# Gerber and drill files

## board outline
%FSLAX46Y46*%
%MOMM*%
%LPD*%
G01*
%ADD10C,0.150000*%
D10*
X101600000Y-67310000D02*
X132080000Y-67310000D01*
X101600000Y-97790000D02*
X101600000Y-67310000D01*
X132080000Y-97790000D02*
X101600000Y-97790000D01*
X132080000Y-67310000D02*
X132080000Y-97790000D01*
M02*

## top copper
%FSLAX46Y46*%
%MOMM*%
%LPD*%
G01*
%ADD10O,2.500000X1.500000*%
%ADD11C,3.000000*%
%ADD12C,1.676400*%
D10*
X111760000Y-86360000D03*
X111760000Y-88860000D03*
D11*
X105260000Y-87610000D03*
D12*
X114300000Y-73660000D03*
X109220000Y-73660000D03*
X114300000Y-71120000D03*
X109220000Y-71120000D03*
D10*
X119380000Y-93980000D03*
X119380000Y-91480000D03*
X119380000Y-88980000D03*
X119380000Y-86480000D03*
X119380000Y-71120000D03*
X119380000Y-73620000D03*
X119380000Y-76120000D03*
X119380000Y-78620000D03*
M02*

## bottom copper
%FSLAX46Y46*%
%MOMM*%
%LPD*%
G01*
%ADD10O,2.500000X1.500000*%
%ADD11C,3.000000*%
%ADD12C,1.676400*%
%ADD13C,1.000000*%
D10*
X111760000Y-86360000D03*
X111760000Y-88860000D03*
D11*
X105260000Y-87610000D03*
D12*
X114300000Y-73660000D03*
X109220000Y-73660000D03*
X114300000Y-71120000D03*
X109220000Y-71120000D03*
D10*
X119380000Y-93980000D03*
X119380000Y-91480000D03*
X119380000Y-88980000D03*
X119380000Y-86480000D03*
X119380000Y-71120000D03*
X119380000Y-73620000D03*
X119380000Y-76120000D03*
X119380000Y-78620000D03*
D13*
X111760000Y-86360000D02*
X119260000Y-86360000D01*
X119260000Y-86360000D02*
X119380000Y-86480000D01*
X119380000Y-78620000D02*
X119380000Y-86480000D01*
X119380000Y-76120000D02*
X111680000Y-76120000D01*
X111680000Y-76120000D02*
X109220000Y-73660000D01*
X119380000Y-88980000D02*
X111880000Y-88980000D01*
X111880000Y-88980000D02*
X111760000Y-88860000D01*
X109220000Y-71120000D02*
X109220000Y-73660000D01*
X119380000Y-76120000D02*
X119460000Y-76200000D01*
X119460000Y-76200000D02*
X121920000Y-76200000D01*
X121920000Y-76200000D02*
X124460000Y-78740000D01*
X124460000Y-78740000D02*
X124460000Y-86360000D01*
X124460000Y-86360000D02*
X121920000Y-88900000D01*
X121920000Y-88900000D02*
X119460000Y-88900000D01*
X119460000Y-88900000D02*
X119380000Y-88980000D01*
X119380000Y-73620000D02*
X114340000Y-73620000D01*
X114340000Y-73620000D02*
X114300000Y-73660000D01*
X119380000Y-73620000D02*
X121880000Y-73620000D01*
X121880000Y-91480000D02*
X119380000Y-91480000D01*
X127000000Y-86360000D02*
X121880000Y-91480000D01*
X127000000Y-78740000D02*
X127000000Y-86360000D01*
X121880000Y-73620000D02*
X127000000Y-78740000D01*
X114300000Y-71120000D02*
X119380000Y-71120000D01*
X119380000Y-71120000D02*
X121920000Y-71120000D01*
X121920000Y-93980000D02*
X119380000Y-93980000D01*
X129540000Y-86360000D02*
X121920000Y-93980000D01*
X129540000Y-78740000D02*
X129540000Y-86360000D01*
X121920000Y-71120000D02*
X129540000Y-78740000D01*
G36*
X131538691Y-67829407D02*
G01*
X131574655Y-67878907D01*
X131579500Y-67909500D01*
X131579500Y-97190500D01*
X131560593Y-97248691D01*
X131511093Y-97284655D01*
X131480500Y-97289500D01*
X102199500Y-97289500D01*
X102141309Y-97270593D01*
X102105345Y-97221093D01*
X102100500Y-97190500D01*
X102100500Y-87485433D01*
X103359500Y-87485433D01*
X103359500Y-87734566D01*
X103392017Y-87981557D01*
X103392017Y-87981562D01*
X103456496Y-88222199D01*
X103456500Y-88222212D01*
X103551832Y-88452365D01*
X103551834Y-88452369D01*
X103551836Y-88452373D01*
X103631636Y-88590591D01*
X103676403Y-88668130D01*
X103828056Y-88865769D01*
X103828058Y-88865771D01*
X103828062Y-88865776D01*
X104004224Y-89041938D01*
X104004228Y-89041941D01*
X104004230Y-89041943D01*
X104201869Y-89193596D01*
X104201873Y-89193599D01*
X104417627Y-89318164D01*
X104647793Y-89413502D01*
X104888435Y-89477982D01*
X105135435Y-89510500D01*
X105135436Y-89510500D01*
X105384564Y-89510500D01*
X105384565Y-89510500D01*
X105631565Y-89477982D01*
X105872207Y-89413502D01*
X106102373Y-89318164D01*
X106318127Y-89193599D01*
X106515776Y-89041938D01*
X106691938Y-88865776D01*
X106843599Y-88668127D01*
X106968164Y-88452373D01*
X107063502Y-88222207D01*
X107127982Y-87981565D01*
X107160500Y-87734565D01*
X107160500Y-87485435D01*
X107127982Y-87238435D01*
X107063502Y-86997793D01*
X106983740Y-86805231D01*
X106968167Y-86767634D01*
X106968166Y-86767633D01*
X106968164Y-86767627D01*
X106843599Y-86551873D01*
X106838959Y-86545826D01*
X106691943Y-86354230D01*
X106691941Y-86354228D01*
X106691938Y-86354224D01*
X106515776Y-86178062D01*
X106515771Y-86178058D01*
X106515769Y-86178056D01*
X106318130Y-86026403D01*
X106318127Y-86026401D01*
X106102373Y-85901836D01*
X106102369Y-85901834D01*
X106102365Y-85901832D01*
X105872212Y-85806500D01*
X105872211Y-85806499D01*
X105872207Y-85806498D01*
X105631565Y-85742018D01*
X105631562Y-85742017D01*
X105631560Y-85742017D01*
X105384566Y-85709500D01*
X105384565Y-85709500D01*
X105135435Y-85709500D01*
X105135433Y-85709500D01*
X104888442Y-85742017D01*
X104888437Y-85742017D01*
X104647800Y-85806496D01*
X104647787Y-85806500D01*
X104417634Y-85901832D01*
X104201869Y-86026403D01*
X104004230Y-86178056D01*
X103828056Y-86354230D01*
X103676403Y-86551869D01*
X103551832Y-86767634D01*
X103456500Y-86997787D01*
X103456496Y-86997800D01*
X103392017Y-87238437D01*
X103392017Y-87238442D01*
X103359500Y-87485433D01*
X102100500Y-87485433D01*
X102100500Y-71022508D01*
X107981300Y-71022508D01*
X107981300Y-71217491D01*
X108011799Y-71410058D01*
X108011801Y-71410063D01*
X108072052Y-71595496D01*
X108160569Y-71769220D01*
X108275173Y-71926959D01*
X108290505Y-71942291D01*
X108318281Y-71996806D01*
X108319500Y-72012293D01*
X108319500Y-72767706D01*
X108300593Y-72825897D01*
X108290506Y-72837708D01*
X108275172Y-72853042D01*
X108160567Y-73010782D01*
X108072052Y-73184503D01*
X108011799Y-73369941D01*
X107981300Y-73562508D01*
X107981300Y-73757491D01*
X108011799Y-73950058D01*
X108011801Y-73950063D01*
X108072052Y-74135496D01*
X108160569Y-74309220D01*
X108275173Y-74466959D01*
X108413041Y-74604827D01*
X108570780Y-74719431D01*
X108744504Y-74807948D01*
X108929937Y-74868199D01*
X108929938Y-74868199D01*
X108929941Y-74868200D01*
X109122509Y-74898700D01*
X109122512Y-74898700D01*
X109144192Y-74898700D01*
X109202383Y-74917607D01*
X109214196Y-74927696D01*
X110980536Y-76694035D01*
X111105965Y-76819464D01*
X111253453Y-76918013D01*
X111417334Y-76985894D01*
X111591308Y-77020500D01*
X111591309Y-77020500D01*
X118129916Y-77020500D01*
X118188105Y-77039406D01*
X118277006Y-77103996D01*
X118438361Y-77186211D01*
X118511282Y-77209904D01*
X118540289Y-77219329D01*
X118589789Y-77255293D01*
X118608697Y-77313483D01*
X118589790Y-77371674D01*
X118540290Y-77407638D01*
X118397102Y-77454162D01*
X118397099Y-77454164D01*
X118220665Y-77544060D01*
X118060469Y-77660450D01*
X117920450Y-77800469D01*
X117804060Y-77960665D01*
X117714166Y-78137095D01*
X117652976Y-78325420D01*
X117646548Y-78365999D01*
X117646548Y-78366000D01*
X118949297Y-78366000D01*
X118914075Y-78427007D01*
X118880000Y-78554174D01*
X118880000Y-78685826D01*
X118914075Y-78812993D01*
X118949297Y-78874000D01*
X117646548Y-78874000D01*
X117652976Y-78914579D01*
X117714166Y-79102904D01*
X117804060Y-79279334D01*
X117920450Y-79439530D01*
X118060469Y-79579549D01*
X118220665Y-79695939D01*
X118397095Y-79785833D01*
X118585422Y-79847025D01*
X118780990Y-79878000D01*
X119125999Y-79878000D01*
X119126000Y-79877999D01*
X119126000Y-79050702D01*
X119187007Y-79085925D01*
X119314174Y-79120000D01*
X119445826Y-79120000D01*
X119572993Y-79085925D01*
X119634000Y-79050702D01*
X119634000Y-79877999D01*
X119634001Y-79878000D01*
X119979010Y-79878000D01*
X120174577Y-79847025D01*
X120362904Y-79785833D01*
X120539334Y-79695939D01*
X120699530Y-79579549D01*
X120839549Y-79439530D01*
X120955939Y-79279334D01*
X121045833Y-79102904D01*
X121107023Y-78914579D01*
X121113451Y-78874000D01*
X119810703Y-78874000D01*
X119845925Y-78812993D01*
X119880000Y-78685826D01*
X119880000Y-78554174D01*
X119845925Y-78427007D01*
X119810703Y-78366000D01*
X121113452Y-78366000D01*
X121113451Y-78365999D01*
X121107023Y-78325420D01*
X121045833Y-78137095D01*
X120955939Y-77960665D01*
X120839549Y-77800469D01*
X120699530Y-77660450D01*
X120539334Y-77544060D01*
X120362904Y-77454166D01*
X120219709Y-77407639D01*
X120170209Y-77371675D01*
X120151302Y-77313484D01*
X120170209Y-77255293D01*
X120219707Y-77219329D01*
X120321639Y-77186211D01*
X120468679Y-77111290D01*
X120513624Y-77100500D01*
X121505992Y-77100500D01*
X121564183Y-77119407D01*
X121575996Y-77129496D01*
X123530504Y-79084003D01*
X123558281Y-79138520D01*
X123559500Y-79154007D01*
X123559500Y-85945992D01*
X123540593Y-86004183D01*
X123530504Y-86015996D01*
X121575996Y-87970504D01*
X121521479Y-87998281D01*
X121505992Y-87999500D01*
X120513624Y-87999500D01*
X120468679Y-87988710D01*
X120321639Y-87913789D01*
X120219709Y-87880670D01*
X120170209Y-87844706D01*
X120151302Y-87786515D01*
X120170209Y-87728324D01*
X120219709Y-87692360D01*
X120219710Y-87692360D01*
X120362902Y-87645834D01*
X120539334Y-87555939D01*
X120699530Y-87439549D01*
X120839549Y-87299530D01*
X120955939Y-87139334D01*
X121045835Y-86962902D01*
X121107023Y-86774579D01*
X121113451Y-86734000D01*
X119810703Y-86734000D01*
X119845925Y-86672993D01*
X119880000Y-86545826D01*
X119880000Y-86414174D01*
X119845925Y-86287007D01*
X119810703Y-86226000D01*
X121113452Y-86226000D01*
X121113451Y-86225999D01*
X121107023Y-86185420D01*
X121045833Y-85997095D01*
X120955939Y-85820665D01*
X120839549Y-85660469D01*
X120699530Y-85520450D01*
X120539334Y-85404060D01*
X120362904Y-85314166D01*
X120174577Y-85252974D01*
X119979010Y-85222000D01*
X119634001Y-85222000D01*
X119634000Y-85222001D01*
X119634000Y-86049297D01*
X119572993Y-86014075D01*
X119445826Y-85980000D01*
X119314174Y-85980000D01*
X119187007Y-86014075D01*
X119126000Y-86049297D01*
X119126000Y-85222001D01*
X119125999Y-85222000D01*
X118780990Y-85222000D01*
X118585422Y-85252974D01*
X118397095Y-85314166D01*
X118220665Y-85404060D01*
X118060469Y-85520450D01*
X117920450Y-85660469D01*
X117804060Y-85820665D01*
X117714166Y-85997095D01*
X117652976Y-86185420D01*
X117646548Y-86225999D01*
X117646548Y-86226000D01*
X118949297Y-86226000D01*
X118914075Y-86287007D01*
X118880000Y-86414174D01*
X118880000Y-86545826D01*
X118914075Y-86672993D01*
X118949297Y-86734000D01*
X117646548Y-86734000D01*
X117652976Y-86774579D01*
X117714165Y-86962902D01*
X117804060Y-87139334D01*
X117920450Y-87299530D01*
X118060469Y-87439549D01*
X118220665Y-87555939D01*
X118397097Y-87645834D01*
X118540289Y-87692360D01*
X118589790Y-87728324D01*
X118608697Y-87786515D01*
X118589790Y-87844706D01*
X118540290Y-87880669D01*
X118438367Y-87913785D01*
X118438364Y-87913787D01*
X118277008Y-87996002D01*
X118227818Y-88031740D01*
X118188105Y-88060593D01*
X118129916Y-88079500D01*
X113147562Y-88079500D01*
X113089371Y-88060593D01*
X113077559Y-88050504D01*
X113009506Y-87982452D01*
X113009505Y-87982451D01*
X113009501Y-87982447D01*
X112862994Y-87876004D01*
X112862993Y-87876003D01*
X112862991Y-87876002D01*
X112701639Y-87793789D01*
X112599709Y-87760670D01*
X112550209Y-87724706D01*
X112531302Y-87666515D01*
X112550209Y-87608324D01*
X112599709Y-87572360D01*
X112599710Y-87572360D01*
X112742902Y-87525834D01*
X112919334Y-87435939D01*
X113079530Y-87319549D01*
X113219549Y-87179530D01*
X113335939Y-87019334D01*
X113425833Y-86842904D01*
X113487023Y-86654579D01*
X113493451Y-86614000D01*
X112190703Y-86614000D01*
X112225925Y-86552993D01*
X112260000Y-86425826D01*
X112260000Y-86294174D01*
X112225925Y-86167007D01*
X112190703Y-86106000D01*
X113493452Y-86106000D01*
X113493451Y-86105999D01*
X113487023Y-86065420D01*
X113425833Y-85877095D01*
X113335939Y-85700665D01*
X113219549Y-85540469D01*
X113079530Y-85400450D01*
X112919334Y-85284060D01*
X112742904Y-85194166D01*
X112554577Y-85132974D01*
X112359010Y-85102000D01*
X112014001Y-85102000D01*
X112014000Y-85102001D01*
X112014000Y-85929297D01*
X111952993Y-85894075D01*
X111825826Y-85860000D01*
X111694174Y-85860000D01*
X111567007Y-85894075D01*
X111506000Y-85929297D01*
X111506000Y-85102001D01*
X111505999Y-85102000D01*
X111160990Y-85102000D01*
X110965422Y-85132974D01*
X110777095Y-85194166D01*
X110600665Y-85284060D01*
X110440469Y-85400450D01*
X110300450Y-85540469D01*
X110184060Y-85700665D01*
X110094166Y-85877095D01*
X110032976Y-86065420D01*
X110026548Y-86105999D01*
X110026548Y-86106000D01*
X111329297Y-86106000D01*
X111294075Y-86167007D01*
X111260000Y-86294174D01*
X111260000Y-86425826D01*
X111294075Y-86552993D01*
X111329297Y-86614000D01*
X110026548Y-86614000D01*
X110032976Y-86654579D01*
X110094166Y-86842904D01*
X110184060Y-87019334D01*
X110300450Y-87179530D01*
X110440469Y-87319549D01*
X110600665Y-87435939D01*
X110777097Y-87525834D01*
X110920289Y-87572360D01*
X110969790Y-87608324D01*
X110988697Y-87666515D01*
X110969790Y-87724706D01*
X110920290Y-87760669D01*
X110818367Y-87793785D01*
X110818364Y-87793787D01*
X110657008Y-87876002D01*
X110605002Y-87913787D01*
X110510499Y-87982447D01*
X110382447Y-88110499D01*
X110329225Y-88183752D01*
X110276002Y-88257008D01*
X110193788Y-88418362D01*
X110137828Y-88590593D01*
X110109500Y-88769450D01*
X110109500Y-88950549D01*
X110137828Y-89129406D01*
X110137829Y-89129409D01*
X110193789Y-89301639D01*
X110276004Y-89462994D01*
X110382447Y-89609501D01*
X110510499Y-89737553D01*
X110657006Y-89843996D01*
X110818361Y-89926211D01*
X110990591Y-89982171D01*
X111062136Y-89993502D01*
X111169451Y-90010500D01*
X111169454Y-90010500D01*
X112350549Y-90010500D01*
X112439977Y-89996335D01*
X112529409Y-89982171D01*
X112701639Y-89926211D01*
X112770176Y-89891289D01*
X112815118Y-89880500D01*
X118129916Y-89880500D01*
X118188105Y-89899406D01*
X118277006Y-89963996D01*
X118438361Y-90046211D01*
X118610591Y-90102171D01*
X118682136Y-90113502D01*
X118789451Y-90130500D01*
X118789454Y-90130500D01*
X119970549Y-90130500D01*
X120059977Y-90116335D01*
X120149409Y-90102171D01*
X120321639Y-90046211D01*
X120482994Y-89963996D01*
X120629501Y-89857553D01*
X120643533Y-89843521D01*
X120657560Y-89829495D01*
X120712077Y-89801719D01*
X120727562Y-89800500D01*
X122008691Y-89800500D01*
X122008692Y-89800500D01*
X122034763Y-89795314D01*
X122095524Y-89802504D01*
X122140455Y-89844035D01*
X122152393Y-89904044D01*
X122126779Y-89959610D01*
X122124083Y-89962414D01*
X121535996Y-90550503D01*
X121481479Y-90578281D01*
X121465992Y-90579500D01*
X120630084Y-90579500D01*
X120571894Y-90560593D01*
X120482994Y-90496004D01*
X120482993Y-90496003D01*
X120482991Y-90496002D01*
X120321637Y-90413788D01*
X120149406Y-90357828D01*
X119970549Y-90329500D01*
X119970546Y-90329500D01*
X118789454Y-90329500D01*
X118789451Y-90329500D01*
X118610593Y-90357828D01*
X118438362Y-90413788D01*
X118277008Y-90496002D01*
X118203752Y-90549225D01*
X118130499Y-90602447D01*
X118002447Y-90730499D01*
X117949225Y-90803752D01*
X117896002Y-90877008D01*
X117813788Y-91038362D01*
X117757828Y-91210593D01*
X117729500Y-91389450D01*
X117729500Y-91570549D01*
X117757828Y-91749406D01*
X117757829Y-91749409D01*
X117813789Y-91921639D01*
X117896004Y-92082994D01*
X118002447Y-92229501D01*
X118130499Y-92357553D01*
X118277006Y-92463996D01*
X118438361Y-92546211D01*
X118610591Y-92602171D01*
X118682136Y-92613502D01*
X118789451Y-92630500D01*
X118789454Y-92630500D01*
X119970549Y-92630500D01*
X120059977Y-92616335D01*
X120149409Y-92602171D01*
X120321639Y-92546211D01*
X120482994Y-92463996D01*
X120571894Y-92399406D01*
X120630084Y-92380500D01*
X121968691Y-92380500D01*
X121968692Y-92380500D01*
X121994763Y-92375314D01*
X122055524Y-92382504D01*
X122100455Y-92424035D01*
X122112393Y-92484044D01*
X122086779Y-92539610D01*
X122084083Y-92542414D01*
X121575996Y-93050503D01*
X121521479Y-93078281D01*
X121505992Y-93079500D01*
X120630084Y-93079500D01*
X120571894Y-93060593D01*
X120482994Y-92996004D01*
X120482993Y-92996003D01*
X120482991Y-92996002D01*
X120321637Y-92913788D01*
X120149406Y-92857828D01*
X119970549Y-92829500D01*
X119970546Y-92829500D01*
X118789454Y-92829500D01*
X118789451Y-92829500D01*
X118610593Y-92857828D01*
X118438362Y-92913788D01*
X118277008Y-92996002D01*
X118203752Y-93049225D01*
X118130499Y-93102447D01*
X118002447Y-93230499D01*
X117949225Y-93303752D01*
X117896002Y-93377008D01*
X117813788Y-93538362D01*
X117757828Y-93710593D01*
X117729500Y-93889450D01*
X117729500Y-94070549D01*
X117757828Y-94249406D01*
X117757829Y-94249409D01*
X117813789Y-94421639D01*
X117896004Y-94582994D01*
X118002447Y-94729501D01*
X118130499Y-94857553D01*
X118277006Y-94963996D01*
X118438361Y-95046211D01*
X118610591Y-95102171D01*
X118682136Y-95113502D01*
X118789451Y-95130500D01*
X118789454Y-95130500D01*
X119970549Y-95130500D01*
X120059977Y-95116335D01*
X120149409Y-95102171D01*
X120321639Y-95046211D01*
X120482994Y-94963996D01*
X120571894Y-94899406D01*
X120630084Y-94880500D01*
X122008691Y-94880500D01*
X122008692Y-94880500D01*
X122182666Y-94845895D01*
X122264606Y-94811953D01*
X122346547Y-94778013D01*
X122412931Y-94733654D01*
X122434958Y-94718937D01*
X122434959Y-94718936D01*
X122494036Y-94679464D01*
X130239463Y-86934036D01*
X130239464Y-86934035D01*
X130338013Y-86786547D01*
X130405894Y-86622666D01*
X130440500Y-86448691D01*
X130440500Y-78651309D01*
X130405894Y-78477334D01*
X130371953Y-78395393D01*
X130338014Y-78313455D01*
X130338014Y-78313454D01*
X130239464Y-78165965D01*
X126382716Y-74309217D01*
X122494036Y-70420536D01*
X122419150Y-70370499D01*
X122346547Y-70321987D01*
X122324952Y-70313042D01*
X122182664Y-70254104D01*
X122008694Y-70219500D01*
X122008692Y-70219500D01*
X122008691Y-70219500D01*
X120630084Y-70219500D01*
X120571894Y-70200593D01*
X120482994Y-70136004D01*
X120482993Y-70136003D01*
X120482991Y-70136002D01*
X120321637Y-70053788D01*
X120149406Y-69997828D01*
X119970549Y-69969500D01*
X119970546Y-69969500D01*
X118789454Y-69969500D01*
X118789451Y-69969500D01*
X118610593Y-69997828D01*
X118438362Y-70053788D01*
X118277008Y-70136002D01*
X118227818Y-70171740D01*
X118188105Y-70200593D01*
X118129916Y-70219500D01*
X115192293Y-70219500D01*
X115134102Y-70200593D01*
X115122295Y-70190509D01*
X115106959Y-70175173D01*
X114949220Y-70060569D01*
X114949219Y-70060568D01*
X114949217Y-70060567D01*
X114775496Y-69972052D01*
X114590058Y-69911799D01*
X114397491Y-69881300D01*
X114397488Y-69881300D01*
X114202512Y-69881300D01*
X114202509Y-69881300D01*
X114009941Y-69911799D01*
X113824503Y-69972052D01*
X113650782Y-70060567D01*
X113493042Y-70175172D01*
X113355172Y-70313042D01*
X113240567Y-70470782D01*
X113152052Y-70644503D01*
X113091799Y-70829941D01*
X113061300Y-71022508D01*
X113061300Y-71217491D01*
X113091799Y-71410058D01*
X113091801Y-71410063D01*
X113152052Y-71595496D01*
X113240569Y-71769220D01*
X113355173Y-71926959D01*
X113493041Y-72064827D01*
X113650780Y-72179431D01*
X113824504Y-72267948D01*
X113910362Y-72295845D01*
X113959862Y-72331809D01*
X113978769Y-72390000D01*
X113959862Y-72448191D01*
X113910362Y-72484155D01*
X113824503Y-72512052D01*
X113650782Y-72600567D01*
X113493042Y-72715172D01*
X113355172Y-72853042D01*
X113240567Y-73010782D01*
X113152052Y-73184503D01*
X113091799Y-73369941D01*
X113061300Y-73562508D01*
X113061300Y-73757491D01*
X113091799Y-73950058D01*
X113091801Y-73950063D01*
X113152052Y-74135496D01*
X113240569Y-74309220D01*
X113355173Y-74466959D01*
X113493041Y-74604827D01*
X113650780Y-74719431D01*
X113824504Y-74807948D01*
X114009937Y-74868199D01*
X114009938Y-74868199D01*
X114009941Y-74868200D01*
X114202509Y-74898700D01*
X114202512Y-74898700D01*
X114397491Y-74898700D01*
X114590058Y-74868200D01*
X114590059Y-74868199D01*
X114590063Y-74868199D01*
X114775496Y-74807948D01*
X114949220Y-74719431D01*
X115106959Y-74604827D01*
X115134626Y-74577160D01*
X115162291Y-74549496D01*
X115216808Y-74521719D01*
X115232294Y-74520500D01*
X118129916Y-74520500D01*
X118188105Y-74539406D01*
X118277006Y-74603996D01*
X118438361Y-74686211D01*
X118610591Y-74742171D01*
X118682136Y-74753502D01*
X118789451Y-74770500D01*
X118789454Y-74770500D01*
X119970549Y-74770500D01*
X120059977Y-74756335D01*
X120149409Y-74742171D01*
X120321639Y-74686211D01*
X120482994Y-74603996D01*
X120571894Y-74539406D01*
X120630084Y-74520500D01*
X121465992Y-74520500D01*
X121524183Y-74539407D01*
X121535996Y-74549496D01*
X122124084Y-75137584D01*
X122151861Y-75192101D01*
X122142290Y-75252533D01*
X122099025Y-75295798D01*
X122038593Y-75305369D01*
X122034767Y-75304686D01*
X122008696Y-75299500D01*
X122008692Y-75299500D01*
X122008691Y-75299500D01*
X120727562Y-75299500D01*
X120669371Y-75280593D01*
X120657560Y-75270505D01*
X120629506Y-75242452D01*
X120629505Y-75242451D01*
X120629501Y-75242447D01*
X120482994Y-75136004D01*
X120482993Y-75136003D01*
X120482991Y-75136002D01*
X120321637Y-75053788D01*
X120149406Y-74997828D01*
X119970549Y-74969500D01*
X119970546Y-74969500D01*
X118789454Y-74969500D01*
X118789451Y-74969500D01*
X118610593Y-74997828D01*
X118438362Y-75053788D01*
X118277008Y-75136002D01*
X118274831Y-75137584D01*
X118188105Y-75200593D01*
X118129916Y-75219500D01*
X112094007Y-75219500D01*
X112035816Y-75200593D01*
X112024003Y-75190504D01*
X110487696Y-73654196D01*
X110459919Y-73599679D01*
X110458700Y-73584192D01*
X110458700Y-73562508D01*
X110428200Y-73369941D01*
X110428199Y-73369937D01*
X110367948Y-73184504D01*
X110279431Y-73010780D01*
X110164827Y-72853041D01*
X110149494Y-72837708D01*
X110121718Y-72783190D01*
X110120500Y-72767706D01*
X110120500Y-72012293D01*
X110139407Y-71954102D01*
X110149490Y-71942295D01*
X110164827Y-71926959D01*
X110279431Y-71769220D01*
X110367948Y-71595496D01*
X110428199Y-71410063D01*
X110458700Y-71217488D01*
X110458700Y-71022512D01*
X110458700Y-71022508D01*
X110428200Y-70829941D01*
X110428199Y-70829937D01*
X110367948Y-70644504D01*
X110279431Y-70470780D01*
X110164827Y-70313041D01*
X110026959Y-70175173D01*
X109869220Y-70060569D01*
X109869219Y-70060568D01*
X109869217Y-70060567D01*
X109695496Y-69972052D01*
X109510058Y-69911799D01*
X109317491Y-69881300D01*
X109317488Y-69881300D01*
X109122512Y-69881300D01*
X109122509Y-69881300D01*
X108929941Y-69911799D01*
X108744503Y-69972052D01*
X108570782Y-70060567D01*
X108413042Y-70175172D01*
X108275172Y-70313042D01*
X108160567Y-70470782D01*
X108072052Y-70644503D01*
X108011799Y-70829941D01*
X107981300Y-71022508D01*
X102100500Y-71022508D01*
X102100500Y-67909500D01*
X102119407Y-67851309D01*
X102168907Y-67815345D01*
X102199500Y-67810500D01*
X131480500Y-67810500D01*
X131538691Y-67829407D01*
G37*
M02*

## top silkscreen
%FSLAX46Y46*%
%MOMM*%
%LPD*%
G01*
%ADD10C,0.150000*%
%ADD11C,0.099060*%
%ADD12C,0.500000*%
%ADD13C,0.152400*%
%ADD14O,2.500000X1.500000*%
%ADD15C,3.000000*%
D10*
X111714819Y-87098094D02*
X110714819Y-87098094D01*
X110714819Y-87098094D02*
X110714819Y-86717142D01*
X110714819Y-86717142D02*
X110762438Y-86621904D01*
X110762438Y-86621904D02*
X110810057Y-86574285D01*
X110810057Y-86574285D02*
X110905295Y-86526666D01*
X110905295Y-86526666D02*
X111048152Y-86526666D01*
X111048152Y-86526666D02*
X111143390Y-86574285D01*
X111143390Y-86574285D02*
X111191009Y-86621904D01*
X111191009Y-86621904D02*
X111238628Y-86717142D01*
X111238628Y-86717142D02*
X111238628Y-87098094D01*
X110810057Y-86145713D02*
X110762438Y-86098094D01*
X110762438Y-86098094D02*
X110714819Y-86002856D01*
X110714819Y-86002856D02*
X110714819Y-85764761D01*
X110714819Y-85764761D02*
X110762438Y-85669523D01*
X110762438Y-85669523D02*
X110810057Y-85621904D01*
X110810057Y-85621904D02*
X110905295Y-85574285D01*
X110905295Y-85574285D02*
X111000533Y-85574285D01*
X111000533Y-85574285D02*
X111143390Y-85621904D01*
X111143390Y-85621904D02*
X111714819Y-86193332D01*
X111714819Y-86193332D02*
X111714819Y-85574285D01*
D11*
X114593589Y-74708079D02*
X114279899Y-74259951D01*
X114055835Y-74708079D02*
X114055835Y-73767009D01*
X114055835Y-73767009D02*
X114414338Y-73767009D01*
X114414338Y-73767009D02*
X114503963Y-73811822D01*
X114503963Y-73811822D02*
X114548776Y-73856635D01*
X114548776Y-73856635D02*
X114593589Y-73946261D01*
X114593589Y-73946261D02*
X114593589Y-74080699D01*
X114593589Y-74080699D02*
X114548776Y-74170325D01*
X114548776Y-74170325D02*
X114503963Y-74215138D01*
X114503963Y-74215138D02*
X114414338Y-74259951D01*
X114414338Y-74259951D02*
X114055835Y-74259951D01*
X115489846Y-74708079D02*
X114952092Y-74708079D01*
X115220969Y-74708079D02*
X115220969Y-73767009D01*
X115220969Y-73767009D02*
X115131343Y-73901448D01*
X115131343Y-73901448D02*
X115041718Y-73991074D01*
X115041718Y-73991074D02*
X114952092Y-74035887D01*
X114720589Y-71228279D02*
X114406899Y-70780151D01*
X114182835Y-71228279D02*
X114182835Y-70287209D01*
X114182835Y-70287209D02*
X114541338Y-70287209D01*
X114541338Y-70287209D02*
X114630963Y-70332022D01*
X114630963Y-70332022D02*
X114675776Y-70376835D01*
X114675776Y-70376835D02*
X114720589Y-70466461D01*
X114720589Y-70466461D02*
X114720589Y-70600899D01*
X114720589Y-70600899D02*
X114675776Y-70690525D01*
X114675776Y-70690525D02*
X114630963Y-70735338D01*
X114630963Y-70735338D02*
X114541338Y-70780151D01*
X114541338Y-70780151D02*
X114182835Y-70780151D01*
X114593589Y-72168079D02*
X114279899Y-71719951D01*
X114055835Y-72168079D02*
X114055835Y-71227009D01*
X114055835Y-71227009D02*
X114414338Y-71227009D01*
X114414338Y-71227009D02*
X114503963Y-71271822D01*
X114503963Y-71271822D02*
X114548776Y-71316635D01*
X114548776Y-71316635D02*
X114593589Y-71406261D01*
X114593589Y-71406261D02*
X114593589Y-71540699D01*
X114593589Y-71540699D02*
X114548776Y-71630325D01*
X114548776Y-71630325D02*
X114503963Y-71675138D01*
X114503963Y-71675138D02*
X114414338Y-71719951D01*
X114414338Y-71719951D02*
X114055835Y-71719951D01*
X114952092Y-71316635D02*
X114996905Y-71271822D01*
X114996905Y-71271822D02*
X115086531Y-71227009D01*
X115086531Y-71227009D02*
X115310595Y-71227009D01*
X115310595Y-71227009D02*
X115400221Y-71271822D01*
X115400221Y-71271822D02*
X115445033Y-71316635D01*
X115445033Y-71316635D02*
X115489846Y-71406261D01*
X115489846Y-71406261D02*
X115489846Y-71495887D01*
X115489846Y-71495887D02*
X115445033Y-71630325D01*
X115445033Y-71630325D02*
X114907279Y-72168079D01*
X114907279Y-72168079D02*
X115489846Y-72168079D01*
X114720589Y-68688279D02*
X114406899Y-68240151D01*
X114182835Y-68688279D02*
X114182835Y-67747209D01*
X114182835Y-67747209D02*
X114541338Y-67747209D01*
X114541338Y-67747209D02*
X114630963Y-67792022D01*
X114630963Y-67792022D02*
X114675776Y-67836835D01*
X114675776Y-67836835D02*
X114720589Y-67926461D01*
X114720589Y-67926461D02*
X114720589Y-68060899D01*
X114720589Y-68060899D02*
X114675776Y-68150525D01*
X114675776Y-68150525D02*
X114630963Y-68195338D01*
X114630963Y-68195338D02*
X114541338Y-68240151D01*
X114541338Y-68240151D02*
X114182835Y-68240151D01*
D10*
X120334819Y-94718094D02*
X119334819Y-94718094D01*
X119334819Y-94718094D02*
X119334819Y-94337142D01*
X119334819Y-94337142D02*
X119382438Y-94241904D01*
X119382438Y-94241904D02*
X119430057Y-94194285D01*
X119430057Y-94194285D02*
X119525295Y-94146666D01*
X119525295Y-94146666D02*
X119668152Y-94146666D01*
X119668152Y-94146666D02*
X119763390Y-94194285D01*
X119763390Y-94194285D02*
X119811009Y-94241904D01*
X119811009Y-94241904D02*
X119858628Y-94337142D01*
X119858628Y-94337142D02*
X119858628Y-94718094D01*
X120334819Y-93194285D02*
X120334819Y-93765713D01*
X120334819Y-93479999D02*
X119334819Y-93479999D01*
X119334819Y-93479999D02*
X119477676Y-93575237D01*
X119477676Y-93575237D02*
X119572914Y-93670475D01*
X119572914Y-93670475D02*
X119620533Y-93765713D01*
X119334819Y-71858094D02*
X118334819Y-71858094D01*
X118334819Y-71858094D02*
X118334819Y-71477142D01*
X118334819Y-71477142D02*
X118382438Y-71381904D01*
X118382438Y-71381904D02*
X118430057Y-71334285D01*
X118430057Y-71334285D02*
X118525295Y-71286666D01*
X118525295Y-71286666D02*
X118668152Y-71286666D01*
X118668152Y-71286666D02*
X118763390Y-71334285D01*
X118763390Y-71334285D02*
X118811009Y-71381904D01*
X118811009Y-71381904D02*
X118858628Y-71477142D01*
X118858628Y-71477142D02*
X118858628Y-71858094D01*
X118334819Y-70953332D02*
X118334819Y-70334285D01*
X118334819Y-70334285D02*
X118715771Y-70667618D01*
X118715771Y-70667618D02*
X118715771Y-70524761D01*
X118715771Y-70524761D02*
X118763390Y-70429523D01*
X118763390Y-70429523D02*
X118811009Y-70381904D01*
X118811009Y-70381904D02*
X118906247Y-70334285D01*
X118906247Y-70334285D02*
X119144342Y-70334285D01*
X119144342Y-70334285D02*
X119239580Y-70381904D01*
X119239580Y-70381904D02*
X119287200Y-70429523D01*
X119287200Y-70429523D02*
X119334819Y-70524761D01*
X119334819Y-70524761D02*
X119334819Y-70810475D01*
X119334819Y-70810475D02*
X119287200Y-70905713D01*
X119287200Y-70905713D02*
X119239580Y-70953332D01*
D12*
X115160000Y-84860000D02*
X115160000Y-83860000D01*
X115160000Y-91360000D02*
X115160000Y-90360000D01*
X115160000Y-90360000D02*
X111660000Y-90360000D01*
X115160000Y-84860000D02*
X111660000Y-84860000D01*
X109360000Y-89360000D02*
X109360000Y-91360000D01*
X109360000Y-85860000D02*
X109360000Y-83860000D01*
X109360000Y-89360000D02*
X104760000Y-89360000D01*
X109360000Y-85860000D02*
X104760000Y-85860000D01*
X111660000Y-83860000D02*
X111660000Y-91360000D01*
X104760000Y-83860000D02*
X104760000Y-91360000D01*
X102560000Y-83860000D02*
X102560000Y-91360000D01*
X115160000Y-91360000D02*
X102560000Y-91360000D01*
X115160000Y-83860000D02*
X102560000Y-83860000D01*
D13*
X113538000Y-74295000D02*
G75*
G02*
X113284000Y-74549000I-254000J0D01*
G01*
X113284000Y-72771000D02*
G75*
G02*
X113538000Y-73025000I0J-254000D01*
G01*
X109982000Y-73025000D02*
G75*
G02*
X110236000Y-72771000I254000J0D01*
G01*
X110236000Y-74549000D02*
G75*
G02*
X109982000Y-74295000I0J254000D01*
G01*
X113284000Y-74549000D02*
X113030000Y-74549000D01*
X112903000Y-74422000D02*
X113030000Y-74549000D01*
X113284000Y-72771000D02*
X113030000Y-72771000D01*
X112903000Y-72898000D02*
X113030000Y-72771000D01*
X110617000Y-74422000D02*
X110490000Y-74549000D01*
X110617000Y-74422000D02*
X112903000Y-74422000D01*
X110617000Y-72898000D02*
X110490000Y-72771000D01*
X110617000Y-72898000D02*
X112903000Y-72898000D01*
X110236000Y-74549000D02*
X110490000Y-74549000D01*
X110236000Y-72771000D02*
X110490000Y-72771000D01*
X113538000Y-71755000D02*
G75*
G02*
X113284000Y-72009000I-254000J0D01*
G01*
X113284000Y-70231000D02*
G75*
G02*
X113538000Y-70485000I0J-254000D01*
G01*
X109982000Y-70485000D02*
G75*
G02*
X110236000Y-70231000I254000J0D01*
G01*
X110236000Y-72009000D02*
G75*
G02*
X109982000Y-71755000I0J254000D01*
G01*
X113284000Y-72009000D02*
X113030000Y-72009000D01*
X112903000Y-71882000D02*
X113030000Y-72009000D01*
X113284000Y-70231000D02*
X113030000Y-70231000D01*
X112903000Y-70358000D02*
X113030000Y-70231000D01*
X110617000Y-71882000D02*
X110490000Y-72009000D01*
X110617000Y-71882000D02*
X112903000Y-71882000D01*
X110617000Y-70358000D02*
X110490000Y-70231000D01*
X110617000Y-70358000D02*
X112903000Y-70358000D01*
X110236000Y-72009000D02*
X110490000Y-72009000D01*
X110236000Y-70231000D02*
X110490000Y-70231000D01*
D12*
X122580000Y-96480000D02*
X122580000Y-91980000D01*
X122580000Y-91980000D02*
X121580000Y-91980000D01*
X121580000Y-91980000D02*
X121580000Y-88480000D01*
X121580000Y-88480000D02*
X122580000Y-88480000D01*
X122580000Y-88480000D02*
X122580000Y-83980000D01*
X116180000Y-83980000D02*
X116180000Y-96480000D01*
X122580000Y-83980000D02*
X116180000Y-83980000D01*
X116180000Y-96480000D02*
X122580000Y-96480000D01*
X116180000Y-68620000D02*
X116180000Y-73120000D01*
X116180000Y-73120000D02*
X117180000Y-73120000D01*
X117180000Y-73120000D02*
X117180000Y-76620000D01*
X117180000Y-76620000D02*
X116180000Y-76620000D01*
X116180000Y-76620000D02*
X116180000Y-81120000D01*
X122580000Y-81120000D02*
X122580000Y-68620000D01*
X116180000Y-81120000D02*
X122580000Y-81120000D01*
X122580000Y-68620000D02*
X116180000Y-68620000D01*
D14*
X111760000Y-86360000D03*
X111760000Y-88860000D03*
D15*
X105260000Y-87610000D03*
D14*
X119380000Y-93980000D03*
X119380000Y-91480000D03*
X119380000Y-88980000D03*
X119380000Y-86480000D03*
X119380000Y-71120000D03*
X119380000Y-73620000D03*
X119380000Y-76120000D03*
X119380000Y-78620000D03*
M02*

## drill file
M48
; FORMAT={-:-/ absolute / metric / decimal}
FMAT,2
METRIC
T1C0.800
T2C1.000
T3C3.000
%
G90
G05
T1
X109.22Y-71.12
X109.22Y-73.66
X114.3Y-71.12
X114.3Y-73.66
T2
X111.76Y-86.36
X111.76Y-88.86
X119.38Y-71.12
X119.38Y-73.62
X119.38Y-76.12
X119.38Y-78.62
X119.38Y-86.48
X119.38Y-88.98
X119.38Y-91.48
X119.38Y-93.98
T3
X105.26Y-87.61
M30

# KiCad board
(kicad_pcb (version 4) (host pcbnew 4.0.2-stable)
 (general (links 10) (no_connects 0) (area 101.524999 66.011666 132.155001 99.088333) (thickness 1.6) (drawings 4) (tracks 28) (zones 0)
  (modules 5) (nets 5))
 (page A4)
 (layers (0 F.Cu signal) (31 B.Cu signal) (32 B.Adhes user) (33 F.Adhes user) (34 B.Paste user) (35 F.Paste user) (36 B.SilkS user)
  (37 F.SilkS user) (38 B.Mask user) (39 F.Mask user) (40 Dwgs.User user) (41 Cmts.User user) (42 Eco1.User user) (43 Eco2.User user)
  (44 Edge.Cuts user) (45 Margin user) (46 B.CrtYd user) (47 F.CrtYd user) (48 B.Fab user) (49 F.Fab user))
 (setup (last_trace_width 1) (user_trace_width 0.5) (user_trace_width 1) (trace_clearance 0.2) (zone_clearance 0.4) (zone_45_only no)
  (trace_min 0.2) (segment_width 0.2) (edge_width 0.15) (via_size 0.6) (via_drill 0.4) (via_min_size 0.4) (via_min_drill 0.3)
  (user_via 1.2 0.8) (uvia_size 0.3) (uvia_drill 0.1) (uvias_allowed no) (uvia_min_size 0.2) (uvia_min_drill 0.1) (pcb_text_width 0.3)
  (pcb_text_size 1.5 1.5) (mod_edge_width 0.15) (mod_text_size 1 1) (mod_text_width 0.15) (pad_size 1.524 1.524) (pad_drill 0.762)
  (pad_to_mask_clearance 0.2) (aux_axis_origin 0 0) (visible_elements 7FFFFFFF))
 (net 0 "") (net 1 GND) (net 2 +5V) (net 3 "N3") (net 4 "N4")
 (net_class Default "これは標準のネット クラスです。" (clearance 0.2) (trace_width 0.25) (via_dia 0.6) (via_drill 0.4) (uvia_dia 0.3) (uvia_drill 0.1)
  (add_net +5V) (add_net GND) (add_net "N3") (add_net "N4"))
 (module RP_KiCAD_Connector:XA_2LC (layer F.Cu) (at 111.76 86.36 270)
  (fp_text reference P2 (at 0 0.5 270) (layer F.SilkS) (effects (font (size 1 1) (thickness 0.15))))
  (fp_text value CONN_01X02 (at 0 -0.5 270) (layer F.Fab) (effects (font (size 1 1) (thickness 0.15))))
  (fp_line (start -1.5 -3.4) (end -2.5 -3.4) (layer F.SilkS) (width 0.5))
  (fp_line (start 5 -3.4) (end 4 -3.4) (layer F.SilkS) (width 0.5))
  (fp_line (start 4 -3.4) (end 4 0.1) (layer F.SilkS) (width 0.5))
  (fp_line (start -1.5 -3.4) (end -1.5 0.1) (layer F.SilkS) (width 0.5))
  (fp_line (start 3 2.4) (end 5 2.4) (layer F.SilkS) (width 0.5))
  (fp_line (start -0.5 2.4) (end -2.5 2.4) (layer F.SilkS) (width 0.5))
  (fp_line (start 3 2.4) (end 3 7) (layer F.SilkS) (width 0.5))
  (fp_line (start -0.5 2.4) (end -0.5 7) (layer F.SilkS) (width 0.5))
  (fp_line (start -2.5 0.1) (end 5 0.1) (layer F.SilkS) (width 0.5))
  (fp_line (start -2.5 7) (end 5 7) (layer F.SilkS) (width 0.5))
  (fp_line (start -2.5 9.2) (end 5 9.2) (layer F.SilkS) (width 0.5))
  (fp_line (start 5 -3.4) (end 5 9.2) (layer F.SilkS) (width 0.5))
  (fp_line (start -2.5 -3.4) (end -2.5 9.2) (layer F.SilkS) (width 0.5))
  (pad 1 thru_hole oval (at 0 0 270) (size 1.5 2.5) (drill 1) (layers *.Cu *.Mask F.SilkS) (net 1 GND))
  (pad 2 thru_hole oval (at 2.5 0 270) (size 1.5 2.5) (drill 1) (layers *.Cu *.Mask F.SilkS) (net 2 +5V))
  (pad "" thru_hole circle (at 1.25 6.5 270) (size 3 3) (drill 3) (layers *.Cu *.Mask F.SilkS) (clearance -0.3)))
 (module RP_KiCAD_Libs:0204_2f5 (layer F.Cu) (at 111.76 73.66 180)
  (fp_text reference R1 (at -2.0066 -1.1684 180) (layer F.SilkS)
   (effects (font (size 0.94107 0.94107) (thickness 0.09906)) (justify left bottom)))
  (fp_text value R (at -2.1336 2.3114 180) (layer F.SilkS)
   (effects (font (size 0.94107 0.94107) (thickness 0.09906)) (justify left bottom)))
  (fp_arc (start -1.524 -0.635) (end -1.778 -0.635) (angle 90) (layer F.SilkS) (width 0.1524))
  (fp_arc (start -1.524 0.635) (end -1.778 0.635) (angle -90) (layer F.SilkS) (width 0.1524))
  (fp_arc (start 1.524 0.635) (end 1.524 0.889) (angle -90) (layer F.SilkS) (width 0.1524))
  (fp_arc (start 1.524 -0.635) (end 1.524 -0.889) (angle 90) (layer F.SilkS) (width 0.1524))
  (fp_line (start -1.524 -0.889) (end -1.27 -0.889) (layer F.SilkS) (width 0.1524))
  (fp_line (start -1.143 -0.762) (end -1.27 -0.889) (layer F.SilkS) (width 0.1524))
  (fp_line (start -1.524 0.889) (end -1.27 0.889) (layer F.SilkS) (width 0.1524))
  (fp_line (start -1.143 0.762) (end -1.27 0.889) (layer F.SilkS) (width 0.1524))
  (fp_line (start 1.143 -0.762) (end 1.27 -0.889) (layer F.SilkS) (width 0.1524))
  (fp_line (start 1.143 -0.762) (end -1.143 -0.762) (layer F.SilkS) (width 0.1524))
  (fp_line (start 1.143 0.762) (end 1.27 0.889) (layer F.SilkS) (width 0.1524))
  (fp_line (start 1.143 0.762) (end -1.143 0.762) (layer F.SilkS) (width 0.1524))
  (fp_line (start 1.524 -0.889) (end 1.27 -0.889) (layer F.SilkS) (width 0.1524))
  (fp_line (start 1.524 0.889) (end 1.27 0.889) (layer F.SilkS) (width 0.1524))
  (pad 1 thru_hole circle (at -2.54 0 180) (size 1.6764 1.6764) (drill 0.8) (layers *.Cu *.Mask) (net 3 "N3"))
  (pad 2 thru_hole circle (at 2.54 0 180) (size 1.6764 1.6764) (drill 0.8) (layers *.Cu *.Mask) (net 2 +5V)))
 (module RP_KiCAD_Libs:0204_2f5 (layer F.Cu) (at 111.76 71.12 180)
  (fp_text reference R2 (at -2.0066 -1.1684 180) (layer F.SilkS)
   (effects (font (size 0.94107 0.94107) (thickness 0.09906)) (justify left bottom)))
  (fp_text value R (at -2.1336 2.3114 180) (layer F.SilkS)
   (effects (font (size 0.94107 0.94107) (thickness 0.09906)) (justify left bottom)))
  (fp_arc (start -1.524 -0.635) (end -1.778 -0.635) (angle 90) (layer F.SilkS) (width 0.1524))
  (fp_arc (start -1.524 0.635) (end -1.778 0.635) (angle -90) (layer F.SilkS) (width 0.1524))
  (fp_arc (start 1.524 0.635) (end 1.524 0.889) (angle -90) (layer F.SilkS) (width 0.1524))
  (fp_arc (start 1.524 -0.635) (end 1.524 -0.889) (angle 90) (layer F.SilkS) (width 0.1524))
  (fp_line (start -1.524 -0.889) (end -1.27 -0.889) (layer F.SilkS) (width 0.1524))
  (fp_line (start -1.143 -0.762) (end -1.27 -0.889) (layer F.SilkS) (width 0.1524))
  (fp_line (start -1.524 0.889) (end -1.27 0.889) (layer F.SilkS) (width 0.1524))
  (fp_line (start -1.143 0.762) (end -1.27 0.889) (layer F.SilkS) (width 0.1524))
  (fp_line (start 1.143 -0.762) (end 1.27 -0.889) (layer F.SilkS) (width 0.1524))
  (fp_line (start 1.143 -0.762) (end -1.143 -0.762) (layer F.SilkS) (width 0.1524))
  (fp_line (start 1.143 0.762) (end 1.27 0.889) (layer F.SilkS) (width 0.1524))
  (fp_line (start 1.143 0.762) (end -1.143 0.762) (layer F.SilkS) (width 0.1524))
  (fp_line (start 1.524 -0.889) (end 1.27 -0.889) (layer F.SilkS) (width 0.1524))
  (fp_line (start 1.524 0.889) (end 1.27 0.889) (layer F.SilkS) (width 0.1524))
  (pad 1 thru_hole circle (at -2.54 0 180) (size 1.6764 1.6764) (drill 0.8) (layers *.Cu *.Mask) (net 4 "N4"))
  (pad 2 thru_hole circle (at 2.54 0 180) (size 1.6764 1.6764) (drill 0.8) (layers *.Cu *.Mask) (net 2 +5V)))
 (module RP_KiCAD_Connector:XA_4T (layer F.Cu) (at 119.38 93.98 90)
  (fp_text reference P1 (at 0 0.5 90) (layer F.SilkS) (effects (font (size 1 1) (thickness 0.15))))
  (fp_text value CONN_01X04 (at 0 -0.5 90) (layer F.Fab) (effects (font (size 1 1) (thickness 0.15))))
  (fp_line (start -2.5 3.2) (end 2 3.2) (layer F.SilkS) (width 0.5))
  (fp_line (start 2 3.2) (end 2 2.2) (layer F.SilkS) (width 0.5))
  (fp_line (start 2 2.2) (end 5.5 2.2) (layer F.SilkS) (width 0.5))
  (fp_line (start 5.5 2.2) (end 5.5 3.2) (layer F.SilkS) (width 0.5))
  (fp_line (start 5.5 3.2) (end 10 3.2) (layer F.SilkS) (width 0.5))
  (fp_line (start 10 -3.2) (end -2.5 -3.2) (layer F.SilkS) (width 0.5))
  (fp_line (start 10 3.2) (end 10 -3.2) (layer F.SilkS) (width 0.5))
  (fp_line (start -2.5 -3.2) (end -2.5 3.2) (layer F.SilkS) (width 0.5))
  (pad 4 thru_hole oval (at 0 0 90) (size 1.5 2.5) (drill 1) (layers *.Cu *.Mask F.SilkS) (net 4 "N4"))
  (pad 3 thru_hole oval (at 2.5 0 90) (size 1.5 2.5) (drill 1) (layers *.Cu *.Mask F.SilkS) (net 3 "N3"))
  (pad 2 thru_hole oval (at 5 0 90) (size 1.5 2.5) (drill 1) (layers *.Cu *.Mask F.SilkS) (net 2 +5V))
  (pad 1 thru_hole oval (at 7.5 0 90) (size 1.5 2.5) (drill 1) (layers *.Cu *.Mask F.SilkS) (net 1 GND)))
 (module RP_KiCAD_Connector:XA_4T (layer F.Cu) (at 119.38 71.12 270)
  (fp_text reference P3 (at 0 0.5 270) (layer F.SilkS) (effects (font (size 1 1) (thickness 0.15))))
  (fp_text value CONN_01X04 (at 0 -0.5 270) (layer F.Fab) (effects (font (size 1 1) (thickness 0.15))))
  (fp_line (start -2.5 3.2) (end 2 3.2) (layer F.SilkS) (width 0.5))
  (fp_line (start 2 3.2) (end 2 2.2) (layer F.SilkS) (width 0.5))
  (fp_line (start 2 2.2) (end 5.5 2.2) (layer F.SilkS) (width 0.5))
  (fp_line (start 5.5 2.2) (end 5.5 3.2) (layer F.SilkS) (width 0.5))
  (fp_line (start 5.5 3.2) (end 10 3.2) (layer F.SilkS) (width 0.5))
  (fp_line (start 10 -3.2) (end -2.5 -3.2) (layer F.SilkS) (width 0.5))
  (fp_line (start 10 3.2) (end 10 -3.2) (layer F.SilkS) (width 0.5))
  (fp_line (start -2.5 -3.2) (end -2.5 3.2) (layer F.SilkS) (width 0.5))
  (pad 4 thru_hole oval (at 0 0 270) (size 1.5 2.5) (drill 1) (layers *.Cu *.Mask F.SilkS) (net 4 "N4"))
  (pad 3 thru_hole oval (at 2.5 0 270) (size 1.5 2.5) (drill 1) (layers *.Cu *.Mask F.SilkS) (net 3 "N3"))
  (pad 2 thru_hole oval (at 5 0 270) (size 1.5 2.5) (drill 1) (layers *.Cu *.Mask F.SilkS) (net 2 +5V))
  (pad 1 thru_hole oval (at 7.5 0 270) (size 1.5 2.5) (drill 1) (layers *.Cu *.Mask F.SilkS) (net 1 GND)))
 (gr_line (start 101.6 67.31) (end 132.08 67.31) (angle 90) (layer Edge.Cuts) (width 0.15))
 (gr_line (start 101.6 97.79) (end 101.6 67.31) (angle 90) (layer Edge.Cuts) (width 0.15))
 (gr_line (start 132.08 97.79) (end 101.6 97.79) (angle 90) (layer Edge.Cuts) (width 0.15))
 (gr_line (start 132.08 67.31) (end 132.08 97.79) (angle 90) (layer Edge.Cuts) (width 0.15))
 (segment (start 111.76 86.36) (end 119.26 86.36) (width 1) (layer B.Cu) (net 1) (status C00000))
 (segment (start 119.26 86.36) (end 119.38 86.48) (width 1) (layer B.Cu) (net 1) (status C00000))
 (segment (start 119.38 78.62) (end 119.38 86.48) (width 1) (layer B.Cu) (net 1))
 (segment (start 119.38 76.12) (end 111.68 76.12) (width 1) (layer B.Cu) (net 2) (status 400000))
 (segment (start 111.68 76.12) (end 109.22 73.66) (width 1) (layer B.Cu) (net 2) (status 800000))
 (segment (start 119.38 88.98) (end 111.88 88.98) (width 1) (layer B.Cu) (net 2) (status C00000))
 (segment (start 111.88 88.98) (end 111.76 88.86) (width 1) (layer B.Cu) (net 2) (status C00000))
 (segment (start 109.22 71.12) (end 109.22 73.66) (width 1) (layer B.Cu) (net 2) (status C00000))
 (segment (start 119.38 76.12) (end 119.46 76.2) (width 1) (layer B.Cu) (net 2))
 (segment (start 119.46 76.2) (end 121.92 76.2) (width 1) (layer B.Cu) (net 2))
 (segment (start 121.92 76.2) (end 124.46 78.74) (width 1) (layer B.Cu) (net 2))
 (segment (start 124.46 78.74) (end 124.46 86.36) (width 1) (layer B.Cu) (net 2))
 (segment (start 124.46 86.36) (end 121.92 88.9) (width 1) (layer B.Cu) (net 2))
 (segment (start 121.92 88.9) (end 119.46 88.9) (width 1) (layer B.Cu) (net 2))
 (segment (start 119.46 88.9) (end 119.38 88.98) (width 1) (layer B.Cu) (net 2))
 (segment (start 119.38 73.62) (end 114.34 73.62) (width 1) (layer B.Cu) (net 3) (status C00000))
 (segment (start 114.34 73.62) (end 114.3 73.66) (width 1) (layer B.Cu) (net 3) (status C00000))
 (segment (start 119.38 73.62) (end 121.88 73.62) (width 1) (layer B.Cu) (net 3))
 (segment (start 121.88 91.48) (end 119.38 91.48) (width 1) (layer B.Cu) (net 3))
 (segment (start 127 86.36) (end 121.88 91.48) (width 1) (layer B.Cu) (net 3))
 (segment (start 127 78.74) (end 127 86.36) (width 1) (layer B.Cu) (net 3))
 (segment (start 121.88 73.62) (end 127 78.74) (width 1) (layer B.Cu) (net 3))
 (segment (start 114.3 71.12) (end 119.38 71.12) (width 1) (layer B.Cu) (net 4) (status C00000))
 (segment (start 119.38 71.12) (end 121.92 71.12) (width 1) (layer B.Cu) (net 4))
 (segment (start 121.92 93.98) (end 119.38 93.98) (width 1) (layer B.Cu) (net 4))
 (segment (start 129.54 86.36) (end 121.92 93.98) (width 1) (layer B.Cu) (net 4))
 (segment (start 129.54 78.74) (end 129.54 86.36) (width 1) (layer B.Cu) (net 4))
 (segment (start 121.92 71.12) (end 129.54 78.74) (width 1) (layer B.Cu) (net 4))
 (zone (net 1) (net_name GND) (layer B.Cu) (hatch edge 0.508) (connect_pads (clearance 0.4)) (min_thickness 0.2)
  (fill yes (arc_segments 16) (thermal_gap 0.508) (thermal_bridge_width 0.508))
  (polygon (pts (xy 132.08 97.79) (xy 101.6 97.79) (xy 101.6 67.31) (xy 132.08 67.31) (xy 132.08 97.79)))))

